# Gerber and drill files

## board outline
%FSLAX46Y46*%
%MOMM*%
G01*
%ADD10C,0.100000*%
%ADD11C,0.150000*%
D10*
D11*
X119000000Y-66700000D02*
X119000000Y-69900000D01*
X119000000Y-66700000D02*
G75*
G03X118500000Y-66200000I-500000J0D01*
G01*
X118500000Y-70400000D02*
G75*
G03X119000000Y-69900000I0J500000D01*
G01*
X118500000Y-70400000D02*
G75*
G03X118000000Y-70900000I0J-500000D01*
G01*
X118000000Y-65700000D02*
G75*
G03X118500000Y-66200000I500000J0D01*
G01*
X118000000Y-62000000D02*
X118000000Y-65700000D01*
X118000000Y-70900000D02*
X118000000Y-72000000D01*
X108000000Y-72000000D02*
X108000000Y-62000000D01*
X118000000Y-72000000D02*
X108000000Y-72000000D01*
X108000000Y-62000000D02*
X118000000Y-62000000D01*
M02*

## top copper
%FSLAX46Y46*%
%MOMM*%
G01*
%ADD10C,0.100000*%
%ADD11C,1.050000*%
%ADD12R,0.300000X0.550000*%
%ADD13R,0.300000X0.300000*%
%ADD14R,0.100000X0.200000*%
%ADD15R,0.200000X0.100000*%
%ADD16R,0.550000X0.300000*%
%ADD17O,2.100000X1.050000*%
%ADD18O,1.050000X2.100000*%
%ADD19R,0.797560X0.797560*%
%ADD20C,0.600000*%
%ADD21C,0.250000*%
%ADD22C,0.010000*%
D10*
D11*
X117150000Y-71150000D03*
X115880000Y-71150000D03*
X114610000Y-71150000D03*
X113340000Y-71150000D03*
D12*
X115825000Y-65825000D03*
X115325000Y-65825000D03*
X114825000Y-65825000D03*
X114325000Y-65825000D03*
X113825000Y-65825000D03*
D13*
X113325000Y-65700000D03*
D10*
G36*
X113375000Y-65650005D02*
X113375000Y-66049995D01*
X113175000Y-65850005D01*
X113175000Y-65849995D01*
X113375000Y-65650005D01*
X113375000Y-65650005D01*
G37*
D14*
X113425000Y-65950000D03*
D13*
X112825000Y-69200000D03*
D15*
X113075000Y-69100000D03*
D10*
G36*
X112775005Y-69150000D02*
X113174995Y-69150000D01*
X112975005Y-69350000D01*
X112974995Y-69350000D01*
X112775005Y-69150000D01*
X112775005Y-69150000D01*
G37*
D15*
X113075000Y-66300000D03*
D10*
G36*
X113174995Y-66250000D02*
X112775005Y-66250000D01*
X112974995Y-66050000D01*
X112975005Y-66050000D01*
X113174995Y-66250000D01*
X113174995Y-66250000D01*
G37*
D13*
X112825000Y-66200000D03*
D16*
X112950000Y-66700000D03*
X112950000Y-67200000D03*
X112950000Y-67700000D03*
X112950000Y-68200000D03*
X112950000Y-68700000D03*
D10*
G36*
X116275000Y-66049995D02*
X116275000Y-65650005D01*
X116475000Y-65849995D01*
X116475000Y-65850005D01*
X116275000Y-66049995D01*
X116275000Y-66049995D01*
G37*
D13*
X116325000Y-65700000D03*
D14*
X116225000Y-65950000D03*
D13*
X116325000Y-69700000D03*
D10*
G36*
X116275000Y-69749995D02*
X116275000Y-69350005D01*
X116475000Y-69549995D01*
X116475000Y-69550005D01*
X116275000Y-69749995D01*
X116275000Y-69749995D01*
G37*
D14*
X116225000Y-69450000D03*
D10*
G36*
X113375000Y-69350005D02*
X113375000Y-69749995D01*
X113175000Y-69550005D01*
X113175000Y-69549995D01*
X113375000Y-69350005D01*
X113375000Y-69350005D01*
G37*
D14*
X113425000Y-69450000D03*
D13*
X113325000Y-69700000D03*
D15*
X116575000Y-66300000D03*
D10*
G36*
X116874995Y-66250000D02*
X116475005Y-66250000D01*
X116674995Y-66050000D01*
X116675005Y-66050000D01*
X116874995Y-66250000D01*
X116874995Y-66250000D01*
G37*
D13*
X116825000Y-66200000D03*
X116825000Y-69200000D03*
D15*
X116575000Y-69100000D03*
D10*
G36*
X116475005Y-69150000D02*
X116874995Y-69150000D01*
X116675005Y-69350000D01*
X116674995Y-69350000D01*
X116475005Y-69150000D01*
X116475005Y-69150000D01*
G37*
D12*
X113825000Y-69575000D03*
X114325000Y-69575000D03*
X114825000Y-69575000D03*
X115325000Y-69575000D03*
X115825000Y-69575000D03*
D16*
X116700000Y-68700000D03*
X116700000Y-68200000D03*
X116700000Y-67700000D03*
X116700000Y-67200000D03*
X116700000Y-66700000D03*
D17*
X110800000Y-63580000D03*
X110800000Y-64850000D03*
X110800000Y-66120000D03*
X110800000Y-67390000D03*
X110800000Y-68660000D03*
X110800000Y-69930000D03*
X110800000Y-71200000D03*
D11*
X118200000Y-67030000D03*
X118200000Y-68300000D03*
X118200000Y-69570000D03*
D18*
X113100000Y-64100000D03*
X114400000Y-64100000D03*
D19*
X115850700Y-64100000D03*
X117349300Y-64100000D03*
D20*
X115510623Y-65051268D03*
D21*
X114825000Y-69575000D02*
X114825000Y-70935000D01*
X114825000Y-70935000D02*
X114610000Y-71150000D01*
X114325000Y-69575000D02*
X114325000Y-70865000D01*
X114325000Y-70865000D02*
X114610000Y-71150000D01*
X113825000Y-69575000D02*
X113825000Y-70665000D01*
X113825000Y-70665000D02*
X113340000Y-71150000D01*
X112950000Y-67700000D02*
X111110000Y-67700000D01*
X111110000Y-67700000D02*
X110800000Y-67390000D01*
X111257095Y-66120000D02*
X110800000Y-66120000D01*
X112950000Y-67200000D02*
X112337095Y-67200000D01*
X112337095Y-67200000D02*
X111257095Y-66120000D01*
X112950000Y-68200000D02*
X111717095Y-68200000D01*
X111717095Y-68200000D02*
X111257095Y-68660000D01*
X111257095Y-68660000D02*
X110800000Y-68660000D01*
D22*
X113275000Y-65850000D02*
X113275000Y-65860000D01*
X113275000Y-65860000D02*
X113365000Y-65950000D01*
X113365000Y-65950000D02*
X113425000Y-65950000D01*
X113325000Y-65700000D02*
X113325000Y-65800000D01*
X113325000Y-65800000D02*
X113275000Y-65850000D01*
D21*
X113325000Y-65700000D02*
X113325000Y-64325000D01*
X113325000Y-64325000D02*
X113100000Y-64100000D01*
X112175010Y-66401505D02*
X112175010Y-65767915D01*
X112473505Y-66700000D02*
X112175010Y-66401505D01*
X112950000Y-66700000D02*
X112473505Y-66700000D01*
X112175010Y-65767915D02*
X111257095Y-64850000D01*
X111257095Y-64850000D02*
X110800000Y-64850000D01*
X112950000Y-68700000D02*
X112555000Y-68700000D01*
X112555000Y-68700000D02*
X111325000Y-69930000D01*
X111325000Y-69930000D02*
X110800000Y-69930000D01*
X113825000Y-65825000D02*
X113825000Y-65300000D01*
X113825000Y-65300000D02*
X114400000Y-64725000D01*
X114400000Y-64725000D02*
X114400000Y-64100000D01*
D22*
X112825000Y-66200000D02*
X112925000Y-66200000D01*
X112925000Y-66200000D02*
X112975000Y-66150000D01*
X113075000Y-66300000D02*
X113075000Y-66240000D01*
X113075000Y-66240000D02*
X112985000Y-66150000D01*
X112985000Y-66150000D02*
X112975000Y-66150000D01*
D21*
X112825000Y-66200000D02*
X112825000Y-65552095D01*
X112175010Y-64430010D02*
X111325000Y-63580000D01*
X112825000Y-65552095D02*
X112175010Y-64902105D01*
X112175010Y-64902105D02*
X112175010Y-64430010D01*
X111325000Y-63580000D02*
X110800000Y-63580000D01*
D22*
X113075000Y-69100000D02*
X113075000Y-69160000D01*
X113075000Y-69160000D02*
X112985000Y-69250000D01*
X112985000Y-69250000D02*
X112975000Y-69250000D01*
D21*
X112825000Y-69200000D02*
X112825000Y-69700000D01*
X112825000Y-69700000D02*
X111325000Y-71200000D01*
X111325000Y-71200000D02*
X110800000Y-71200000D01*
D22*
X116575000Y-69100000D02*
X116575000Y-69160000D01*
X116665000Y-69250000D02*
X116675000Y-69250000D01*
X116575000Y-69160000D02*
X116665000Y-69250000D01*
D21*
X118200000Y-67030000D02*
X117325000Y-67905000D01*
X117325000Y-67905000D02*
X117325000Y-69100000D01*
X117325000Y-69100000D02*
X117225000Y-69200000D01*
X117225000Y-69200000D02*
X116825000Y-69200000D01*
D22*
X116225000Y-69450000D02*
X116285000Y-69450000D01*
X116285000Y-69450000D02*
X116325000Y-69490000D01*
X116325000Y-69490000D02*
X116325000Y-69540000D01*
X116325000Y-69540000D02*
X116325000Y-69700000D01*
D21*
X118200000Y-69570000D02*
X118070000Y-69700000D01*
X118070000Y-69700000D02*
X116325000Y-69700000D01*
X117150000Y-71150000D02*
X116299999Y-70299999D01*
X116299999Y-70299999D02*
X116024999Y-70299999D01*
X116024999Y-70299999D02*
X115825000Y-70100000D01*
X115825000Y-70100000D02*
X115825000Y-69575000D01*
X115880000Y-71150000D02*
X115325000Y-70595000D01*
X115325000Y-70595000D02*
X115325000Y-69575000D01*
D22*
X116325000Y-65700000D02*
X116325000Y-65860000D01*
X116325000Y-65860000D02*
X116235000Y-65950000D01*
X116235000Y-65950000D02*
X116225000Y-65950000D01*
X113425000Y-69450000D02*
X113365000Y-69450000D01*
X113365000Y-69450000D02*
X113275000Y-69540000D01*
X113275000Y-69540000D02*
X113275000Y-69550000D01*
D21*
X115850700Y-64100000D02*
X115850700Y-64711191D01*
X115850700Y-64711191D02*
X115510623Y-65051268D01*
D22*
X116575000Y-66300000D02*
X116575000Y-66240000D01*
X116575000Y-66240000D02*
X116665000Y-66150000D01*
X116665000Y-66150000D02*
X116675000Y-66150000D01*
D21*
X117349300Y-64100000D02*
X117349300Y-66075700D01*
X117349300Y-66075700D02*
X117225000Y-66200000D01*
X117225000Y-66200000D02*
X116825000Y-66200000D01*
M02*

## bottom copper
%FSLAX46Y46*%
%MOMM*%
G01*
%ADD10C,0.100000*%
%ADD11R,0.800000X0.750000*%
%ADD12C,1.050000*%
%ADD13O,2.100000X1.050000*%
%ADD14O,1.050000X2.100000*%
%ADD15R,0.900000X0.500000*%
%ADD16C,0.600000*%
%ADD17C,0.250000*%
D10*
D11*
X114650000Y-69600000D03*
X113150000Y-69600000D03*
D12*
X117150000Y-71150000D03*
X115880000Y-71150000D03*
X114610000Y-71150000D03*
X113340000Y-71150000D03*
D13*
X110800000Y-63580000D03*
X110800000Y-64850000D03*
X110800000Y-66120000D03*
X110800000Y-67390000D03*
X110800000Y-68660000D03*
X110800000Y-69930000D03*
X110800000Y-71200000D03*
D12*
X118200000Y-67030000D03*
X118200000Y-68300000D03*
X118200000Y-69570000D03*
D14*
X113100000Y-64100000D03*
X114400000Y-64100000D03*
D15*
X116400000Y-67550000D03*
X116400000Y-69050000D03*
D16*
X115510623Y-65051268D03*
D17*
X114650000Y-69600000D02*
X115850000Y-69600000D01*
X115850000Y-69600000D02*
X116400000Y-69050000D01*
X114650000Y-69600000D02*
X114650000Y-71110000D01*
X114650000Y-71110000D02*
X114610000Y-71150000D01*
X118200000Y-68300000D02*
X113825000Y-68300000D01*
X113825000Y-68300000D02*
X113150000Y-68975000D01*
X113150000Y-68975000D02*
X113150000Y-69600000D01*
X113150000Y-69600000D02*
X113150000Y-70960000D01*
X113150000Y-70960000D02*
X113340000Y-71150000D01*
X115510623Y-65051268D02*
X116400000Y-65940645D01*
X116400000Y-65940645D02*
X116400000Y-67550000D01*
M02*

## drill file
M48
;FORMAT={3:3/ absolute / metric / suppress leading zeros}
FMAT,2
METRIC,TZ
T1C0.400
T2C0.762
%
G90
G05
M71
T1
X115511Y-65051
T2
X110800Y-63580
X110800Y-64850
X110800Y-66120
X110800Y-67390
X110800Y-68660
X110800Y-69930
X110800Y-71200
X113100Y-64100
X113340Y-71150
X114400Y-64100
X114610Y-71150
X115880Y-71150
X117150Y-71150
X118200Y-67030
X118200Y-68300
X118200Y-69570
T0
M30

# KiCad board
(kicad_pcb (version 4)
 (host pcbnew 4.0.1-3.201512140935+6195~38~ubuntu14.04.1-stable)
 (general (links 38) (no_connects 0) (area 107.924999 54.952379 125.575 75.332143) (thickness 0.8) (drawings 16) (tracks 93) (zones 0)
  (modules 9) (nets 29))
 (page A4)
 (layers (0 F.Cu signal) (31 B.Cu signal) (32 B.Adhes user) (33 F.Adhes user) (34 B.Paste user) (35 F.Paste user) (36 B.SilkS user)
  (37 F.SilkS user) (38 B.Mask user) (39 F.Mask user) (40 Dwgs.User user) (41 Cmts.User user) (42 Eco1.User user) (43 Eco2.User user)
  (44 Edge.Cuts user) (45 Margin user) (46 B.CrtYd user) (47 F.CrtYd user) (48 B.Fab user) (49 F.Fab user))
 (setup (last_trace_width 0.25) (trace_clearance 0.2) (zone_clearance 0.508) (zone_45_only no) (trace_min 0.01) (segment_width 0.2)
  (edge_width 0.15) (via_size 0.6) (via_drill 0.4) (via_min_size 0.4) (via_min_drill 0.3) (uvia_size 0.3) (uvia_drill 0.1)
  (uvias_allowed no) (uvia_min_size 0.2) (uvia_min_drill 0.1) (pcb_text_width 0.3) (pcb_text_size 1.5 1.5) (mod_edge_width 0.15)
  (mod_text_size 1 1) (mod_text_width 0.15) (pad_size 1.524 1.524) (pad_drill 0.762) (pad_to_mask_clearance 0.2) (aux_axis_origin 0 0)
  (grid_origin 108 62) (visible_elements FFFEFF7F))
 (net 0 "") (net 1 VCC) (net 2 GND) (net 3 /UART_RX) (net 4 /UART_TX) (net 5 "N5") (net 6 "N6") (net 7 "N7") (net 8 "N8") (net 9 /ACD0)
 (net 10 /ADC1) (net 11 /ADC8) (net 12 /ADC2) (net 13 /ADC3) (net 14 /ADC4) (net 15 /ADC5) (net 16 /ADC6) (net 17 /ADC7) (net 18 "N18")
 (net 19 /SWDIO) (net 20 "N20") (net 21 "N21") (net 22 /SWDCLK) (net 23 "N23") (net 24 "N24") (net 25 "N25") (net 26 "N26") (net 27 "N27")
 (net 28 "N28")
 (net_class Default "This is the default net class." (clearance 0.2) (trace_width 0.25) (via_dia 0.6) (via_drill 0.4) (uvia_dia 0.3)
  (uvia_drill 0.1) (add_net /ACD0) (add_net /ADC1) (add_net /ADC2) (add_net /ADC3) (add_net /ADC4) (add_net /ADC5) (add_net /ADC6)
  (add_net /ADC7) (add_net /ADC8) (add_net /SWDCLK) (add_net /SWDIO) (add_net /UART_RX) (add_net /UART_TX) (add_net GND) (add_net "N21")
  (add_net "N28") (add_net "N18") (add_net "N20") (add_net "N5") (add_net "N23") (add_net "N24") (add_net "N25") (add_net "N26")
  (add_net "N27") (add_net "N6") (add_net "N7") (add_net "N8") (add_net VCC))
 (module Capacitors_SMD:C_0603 (layer B.Cu) (at 113.9 69.6 180)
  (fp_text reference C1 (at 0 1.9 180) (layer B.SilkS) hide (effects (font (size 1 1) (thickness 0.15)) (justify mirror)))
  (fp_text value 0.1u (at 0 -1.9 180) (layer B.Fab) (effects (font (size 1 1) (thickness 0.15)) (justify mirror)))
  (pad 1 smd rect (at -0.75 0 180) (size 0.8 0.75) (layers B.Cu B.Paste B.Mask) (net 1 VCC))
  (pad 2 smd rect (at 0.75 0 180) (size 0.8 0.75) (layers B.Cu B.Paste B.Mask) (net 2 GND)))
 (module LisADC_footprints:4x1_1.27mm (layer F.Cu) (at 117.15 71.15)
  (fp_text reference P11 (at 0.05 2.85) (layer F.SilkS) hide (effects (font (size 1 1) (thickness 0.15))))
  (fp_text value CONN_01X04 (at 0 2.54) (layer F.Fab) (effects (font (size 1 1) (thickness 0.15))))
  (pad 1 thru_hole circle (at 0 0) (size 1.05 1.05) (drill 0.762) (layers *.Cu *.Mask F.SilkS) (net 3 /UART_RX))
  (pad 2 thru_hole circle (at -1.27 0) (size 1.05 1.05) (drill 0.762) (layers *.Cu *.Mask F.SilkS) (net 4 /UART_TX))
  (pad 3 thru_hole circle (at -2.54 0) (size 1.05 1.05) (drill 0.762) (layers *.Cu *.Mask F.SilkS) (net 1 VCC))
  (pad 4 thru_hole circle (at -3.81 0) (size 1.05 1.05) (drill 0.762) (layers *.Cu *.Mask F.SilkS) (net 2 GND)))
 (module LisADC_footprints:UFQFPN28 (layer F.Cu) (at 114.825 67.7 270)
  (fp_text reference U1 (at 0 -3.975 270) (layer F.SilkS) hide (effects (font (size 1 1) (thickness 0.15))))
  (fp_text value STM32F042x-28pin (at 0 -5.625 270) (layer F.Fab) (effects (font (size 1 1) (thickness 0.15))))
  (pad 2 smd rect (at -1.875 -1 270) (size 0.55 0.3) (layers F.Cu F.Paste F.Mask) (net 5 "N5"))
  (pad 3 smd rect (at -1.875 -0.5 270) (size 0.55 0.3) (layers F.Cu F.Paste F.Mask) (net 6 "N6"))
  (pad 4 smd rect (at -1.875 0 270) (size 0.55 0.3) (layers F.Cu F.Paste F.Mask) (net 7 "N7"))
  (pad 5 smd rect (at -1.875 0.5 270) (size 0.55 0.3) (layers F.Cu F.Paste F.Mask) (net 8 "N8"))
  (pad 6 smd rect (at -1.875 1 270) (size 0.55 0.3) (layers F.Cu F.Paste F.Mask) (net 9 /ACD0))
  (pad 7 smd rect (at -2 1.5) (size 0.3 0.3) (layers F.Cu F.Paste F.Mask) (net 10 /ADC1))
  (pad 7 smd trapezoid (at -1.85 1.55 180) (size 0.2 0.2) (rect_delta 0.19999 0) (layers F.Cu F.Paste F.Mask) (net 10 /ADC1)
   (solder_mask_margin 0.1))
  (pad 7 smd rect (at -1.75 1.4 270) (size 0.2 0.1) (layers F.Cu F.Paste F.Mask) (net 10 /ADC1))
  (pad 14 smd rect (at 1.5 2 90) (size 0.3 0.3) (layers F.Cu F.Paste F.Mask) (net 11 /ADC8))
  (pad 14 smd rect (at 1.4 1.75) (size 0.2 0.1) (layers F.Cu F.Paste F.Mask) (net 11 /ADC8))
  (pad 14 smd trapezoid (at 1.55 1.85 270) (size 0.2 0.2) (rect_delta 0.19999 0) (layers F.Cu F.Paste F.Mask) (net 11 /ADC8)
   (solder_mask_margin 0.1))
  (pad 8 smd rect (at -1.4 1.75) (size 0.2 0.1) (layers F.Cu F.Paste F.Mask) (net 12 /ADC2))
  (pad 8 smd trapezoid (at -1.55 1.85 90) (size 0.2 0.2) (rect_delta 0.19999 0) (layers F.Cu F.Paste F.Mask) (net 12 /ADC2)
   (solder_mask_margin 0.1))
  (pad 8 smd rect (at -1.5 2 90) (size 0.3 0.3) (layers F.Cu F.Paste F.Mask) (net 12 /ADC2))
  (pad 9 smd rect (at -1 1.875) (size 0.55 0.3) (layers F.Cu F.Paste F.Mask) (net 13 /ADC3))
  (pad 10 smd rect (at -0.5 1.875) (size 0.55 0.3) (layers F.Cu F.Paste F.Mask) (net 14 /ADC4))
  (pad 11 smd rect (at 0 1.875) (size 0.55 0.3) (layers F.Cu F.Paste F.Mask) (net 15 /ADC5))
  (pad 12 smd rect (at 0.5 1.875) (size 0.55 0.3) (layers F.Cu F.Paste F.Mask) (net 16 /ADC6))
  (pad 13 smd rect (at 1 1.875) (size 0.55 0.3) (layers F.Cu F.Paste F.Mask) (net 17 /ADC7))
  (pad 1 smd trapezoid (at -1.85 -1.55) (size 0.2 0.2) (rect_delta 0.19999 0) (layers F.Cu F.Paste F.Mask) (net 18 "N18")
   (solder_mask_margin 0.1))
  (pad 1 smd rect (at -2 -1.5) (size 0.3 0.3) (layers F.Cu F.Paste F.Mask) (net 18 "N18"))
  (pad 1 smd rect (at -1.75 -1.4 270) (size 0.2 0.1) (layers F.Cu F.Paste F.Mask) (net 18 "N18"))
  (pad 21 smd rect (at 2 -1.5 180) (size 0.3 0.3) (layers F.Cu F.Paste F.Mask) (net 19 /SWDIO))
  (pad 21 smd trapezoid (at 1.85 -1.55) (size 0.2 0.2) (rect_delta 0.19999 0) (layers F.Cu F.Paste F.Mask) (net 19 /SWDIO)
   (solder_mask_margin 0.1))
  (pad 21 smd rect (at 1.75 -1.4 90) (size 0.2 0.1) (layers F.Cu F.Paste F.Mask) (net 19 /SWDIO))
  (pad 15 smd trapezoid (at 1.85 1.55 180) (size 0.2 0.2) (rect_delta 0.19999 0) (layers F.Cu F.Paste F.Mask) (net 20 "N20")
   (solder_mask_margin 0.1))
  (pad 15 smd rect (at 1.75 1.4 90) (size 0.2 0.1) (layers F.Cu F.Paste F.Mask) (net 20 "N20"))
  (pad 15 smd rect (at 2 1.5 180) (size 0.3 0.3) (layers F.Cu F.Paste F.Mask) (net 20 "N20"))
  (pad 28 smd rect (at -1.4 -1.75 180) (size 0.2 0.1) (layers F.Cu F.Paste F.Mask) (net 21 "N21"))
  (pad 28 smd trapezoid (at -1.55 -1.85 90) (size 0.2 0.2) (rect_delta 0.19999 0) (layers F.Cu F.Paste F.Mask) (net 21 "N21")
   (solder_mask_margin 0.1))
  (pad 28 smd rect (at -1.5 -2 270) (size 0.3 0.3) (layers F.Cu F.Paste F.Mask) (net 21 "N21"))
  (pad 22 smd rect (at 1.5 -2 270) (size 0.3 0.3) (layers F.Cu F.Paste F.Mask) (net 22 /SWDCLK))
  (pad 22 smd rect (at 1.4 -1.75 180) (size 0.2 0.1) (layers F.Cu F.Paste F.Mask) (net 22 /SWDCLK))
  (pad 22 smd trapezoid (at 1.55 -1.85 270) (size 0.2 0.2) (rect_delta 0.19999 0) (layers F.Cu F.Paste F.Mask) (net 22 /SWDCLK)
   (solder_mask_margin 0.1))
  (pad 16 smd rect (at 1.875 1 90) (size 0.55 0.3) (layers F.Cu F.Paste F.Mask) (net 2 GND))
  (pad 17 smd rect (at 1.875 0.5 90) (size 0.55 0.3) (layers F.Cu F.Paste F.Mask) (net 1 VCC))
  (pad 18 smd rect (at 1.875 0 90) (size 0.55 0.3) (layers F.Cu F.Paste F.Mask) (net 1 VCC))
  (pad 19 smd rect (at 1.875 -0.5 90) (size 0.55 0.3) (layers F.Cu F.Paste F.Mask) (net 4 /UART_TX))
  (pad 20 smd rect (at 1.875 -1 90) (size 0.55 0.3) (layers F.Cu F.Paste F.Mask) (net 3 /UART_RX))
  (pad 23 smd rect (at 1 -1.875 180) (size 0.55 0.3) (layers F.Cu F.Paste F.Mask) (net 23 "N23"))
  (pad 24 smd rect (at 0.5 -1.875 180) (size 0.55 0.3) (layers F.Cu F.Paste F.Mask) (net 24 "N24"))
  (pad 25 smd rect (at 0 -1.875 180) (size 0.55 0.3) (layers F.Cu F.Paste F.Mask) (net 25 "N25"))
  (pad 26 smd rect (at -0.5 -1.875 180) (size 0.55 0.3) (layers F.Cu F.Paste F.Mask) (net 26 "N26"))
  (pad 27 smd rect (at -1 -1.875 180) (size 0.55 0.3) (layers F.Cu F.Paste F.Mask) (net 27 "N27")))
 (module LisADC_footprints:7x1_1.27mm (layer F.Cu) (at 110.8 63.58 90)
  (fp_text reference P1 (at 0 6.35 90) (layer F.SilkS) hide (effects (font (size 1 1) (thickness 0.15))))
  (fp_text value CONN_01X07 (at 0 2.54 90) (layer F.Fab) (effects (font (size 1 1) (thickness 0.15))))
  (pad 1 thru_hole oval (at 0 0 90) (size 1.05 2.1) (drill 0.762) (layers *.Cu *.Mask F.SilkS) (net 12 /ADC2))
  (pad 2 thru_hole oval (at -1.27 0 90) (size 1.05 2.1) (drill 0.762) (layers *.Cu *.Mask F.SilkS) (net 13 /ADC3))
  (pad 3 thru_hole oval (at -2.54 0 90) (size 1.05 2.1) (drill 0.762) (layers *.Cu *.Mask F.SilkS) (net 14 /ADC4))
  (pad 4 thru_hole oval (at -3.81 0 90) (size 1.05 2.1) (drill 0.762) (layers *.Cu *.Mask F.SilkS) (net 15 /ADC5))
  (pad 5 thru_hole oval (at -5.08 0 90) (size 1.05 2.1) (drill 0.762) (layers *.Cu *.Mask F.SilkS) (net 16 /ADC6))
  (pad 6 thru_hole oval (at -6.35 0 90) (size 1.05 2.1) (drill 0.762) (layers *.Cu *.Mask F.SilkS) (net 17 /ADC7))
  (pad 7 thru_hole oval (at -7.62 0 90) (size 1.05 2.1) (drill 0.762) (layers *.Cu *.Mask F.SilkS) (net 11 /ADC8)))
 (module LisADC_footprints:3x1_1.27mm (layer F.Cu) (at 118.25 68.305 90)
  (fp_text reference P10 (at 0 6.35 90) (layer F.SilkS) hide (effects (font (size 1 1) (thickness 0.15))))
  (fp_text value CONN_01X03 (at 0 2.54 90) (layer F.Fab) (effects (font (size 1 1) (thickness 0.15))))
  (pad 1 thru_hole circle (at 1.275 -0.05 90) (size 1.05 1.05) (drill 0.762) (layers *.Cu *.Mask F.SilkS) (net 22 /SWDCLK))
  (pad 2 thru_hole circle (at 0.005 -0.05 90) (size 1.05 1.05) (drill 0.762) (layers *.Cu *.Mask F.SilkS) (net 2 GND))
  (pad 3 thru_hole circle (at -1.265 -0.05 90) (size 1.05 1.05) (drill 0.762) (layers *.Cu *.Mask F.SilkS) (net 19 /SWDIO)))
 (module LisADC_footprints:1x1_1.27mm (layer F.Cu) (at 113.1 64.1)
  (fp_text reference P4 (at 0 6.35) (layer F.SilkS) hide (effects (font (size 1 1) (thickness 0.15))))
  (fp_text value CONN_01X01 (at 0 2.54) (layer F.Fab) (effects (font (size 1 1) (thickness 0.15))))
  (pad 1 thru_hole oval (at 0 0) (size 1.05 2.1) (drill 0.762) (layers *.Cu *.Mask F.SilkS) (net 10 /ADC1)))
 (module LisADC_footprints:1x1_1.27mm (layer F.Cu) (at 114.4 64.1)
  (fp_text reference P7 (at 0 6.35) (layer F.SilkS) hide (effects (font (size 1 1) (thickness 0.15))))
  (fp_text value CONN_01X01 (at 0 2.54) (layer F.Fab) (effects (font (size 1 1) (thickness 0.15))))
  (pad 1 thru_hole oval (at 0 0) (size 1.05 2.1) (drill 0.762) (layers *.Cu *.Mask F.SilkS) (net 9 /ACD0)))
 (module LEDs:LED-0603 (layer F.Cu) (at 116.6 64.1 180)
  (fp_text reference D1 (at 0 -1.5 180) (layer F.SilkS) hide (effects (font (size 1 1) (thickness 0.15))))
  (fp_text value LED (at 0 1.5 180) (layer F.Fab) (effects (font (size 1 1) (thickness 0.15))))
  (pad 2 smd rect (at 0.7493 0) (size 0.79756 0.79756) (layers F.Cu F.Paste F.Mask) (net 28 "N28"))
  (pad 1 smd rect (at -0.7493 0) (size 0.79756 0.79756) (layers F.Cu F.Paste F.Mask) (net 21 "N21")))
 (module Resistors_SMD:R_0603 (layer B.Cu) (at 116.4 68.3 270)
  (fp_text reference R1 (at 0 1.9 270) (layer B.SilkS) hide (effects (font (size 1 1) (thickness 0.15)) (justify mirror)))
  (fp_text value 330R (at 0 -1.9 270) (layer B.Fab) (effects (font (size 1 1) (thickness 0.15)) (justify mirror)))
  (pad 1 smd rect (at -0.75 0 270) (size 0.5 0.9) (layers B.Cu B.Paste B.Mask) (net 28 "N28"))
  (pad 2 smd rect (at 0.75 0 270) (size 0.5 0.9) (layers B.Cu B.Paste B.Mask) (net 1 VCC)))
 (gr_line (start 119 66.7) (end 119 69.9) (layer Edge.Cuts) (width 0.15))
 (gr_arc (start 118.5 66.7) (end 118.5 66.2) (angle 90) (layer Edge.Cuts) (width 0.15))
 (gr_arc (start 118.5 69.9) (end 119 69.9) (angle 90) (layer Edge.Cuts) (width 0.15))
 (gr_arc (start 118.5 70.9) (end 118 70.9) (angle 90) (layer Edge.Cuts) (width 0.15))
 (gr_arc (start 118.5 65.7) (end 118.5 66.2) (angle 90) (layer Edge.Cuts) (width 0.15))
 (gr_line (start 118 62) (end 118 65.7) (layer Edge.Cuts) (width 0.15))
 (gr_line (start 118 70.9) (end 118 72) (layer Edge.Cuts) (width 0.15))
 (gr_line (start 108 72) (end 108 62) (layer Edge.Cuts) (width 0.15))
 (gr_line (start 118 72) (end 108 72) (layer Edge.Cuts) (width 0.15))
 (gr_line (start 108 62) (end 118 62) (layer Edge.Cuts) (width 0.15))
 (segment (start 114.65 69.6) (end 115.85 69.6) (width 0.25) (layer B.Cu) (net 1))
 (segment (start 115.85 69.6) (end 116.4 69.05) (width 0.25) (layer B.Cu) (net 1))
 (segment (start 114.825 69.575) (end 114.825 70.935) (width 0.25) (layer F.Cu) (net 1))
 (segment (start 114.825 70.935) (end 114.61 71.15) (width 0.25) (layer F.Cu) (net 1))
 (segment (start 114.325 69.575) (end 114.325 70.865) (width 0.25) (layer F.Cu) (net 1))
 (segment (start 114.325 70.865) (end 114.61 71.15) (width 0.25) (layer F.Cu) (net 1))
 (segment (start 114.65 69.6) (end 114.65 71.11) (width 0.25) (layer B.Cu) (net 1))
 (segment (start 114.65 71.11) (end 114.61 71.15) (width 0.25) (layer B.Cu) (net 1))
 (segment (start 118.2 68.3) (end 113.825 68.3) (width 0.25) (layer B.Cu) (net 2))
 (segment (start 113.825 68.3) (end 113.15 68.975) (width 0.25) (layer B.Cu) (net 2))
 (segment (start 113.15 68.975) (end 113.15 69.6) (width 0.25) (layer B.Cu) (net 2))
 (segment (start 113.825 69.575) (end 113.825 70.665) (width 0.25) (layer F.Cu) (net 2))
 (segment (start 113.825 70.665) (end 113.34 71.15) (width 0.25) (layer F.Cu) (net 2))
 (segment (start 113.15 69.6) (end 113.15 70.96) (width 0.25) (layer B.Cu) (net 2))
 (segment (start 113.15 70.96) (end 113.34 71.15) (width 0.25) (layer B.Cu) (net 2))
 (segment (start 112.95 67.7) (end 111.11 67.7) (width 0.25) (layer F.Cu) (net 15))
 (segment (start 111.11 67.7) (end 110.8 67.39) (width 0.25) (layer F.Cu) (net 15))
 (segment (start 111.257095 66.12) (end 110.8 66.12) (width 0.25) (layer F.Cu) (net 14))
 (segment (start 112.95 67.2) (end 112.337095 67.2) (width 0.25) (layer F.Cu) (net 14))
 (segment (start 112.337095 67.2) (end 111.257095 66.12) (width 0.25) (layer F.Cu) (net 14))
 (segment (start 112.95 68.2) (end 111.717095 68.2) (width 0.25) (layer F.Cu) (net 16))
 (segment (start 111.717095 68.2) (end 111.257095 68.66) (width 0.25) (layer F.Cu) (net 16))
 (segment (start 111.257095 68.66) (end 110.8 68.66) (width 0.25) (layer F.Cu) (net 16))
 (segment (start 113.275 65.85) (end 113.275 65.86) (width 0.01) (layer F.Cu) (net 10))
 (segment (start 113.275 65.86) (end 113.365 65.95) (width 0.01) (layer F.Cu) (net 10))
 (segment (start 113.365 65.95) (end 113.425 65.95) (width 0.01) (layer F.Cu) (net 10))
 (segment (start 113.325 65.7) (end 113.325 65.8) (width 0.01) (layer F.Cu) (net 10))
 (segment (start 113.325 65.8) (end 113.275 65.85) (width 0.01) (layer F.Cu) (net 10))
 (segment (start 113.325 65.7) (end 113.325 64.325) (width 0.25) (layer F.Cu) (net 10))
 (segment (start 113.325 64.325) (end 113.1 64.1) (width 0.25) (layer F.Cu) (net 10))
 (segment (start 112.17501 66.401505) (end 112.17501 65.767915) (width 0.25) (layer F.Cu) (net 13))
 (segment (start 112.473505 66.7) (end 112.17501 66.401505) (width 0.25) (layer F.Cu) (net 13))
 (segment (start 112.95 66.7) (end 112.473505 66.7) (width 0.25) (layer F.Cu) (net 13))
 (segment (start 112.17501 65.767915) (end 111.257095 64.85) (width 0.25) (layer F.Cu) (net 13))
 (segment (start 111.257095 64.85) (end 110.8 64.85) (width 0.25) (layer F.Cu) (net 13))
 (segment (start 112.95 68.7) (end 112.555 68.7) (width 0.25) (layer F.Cu) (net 17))
 (segment (start 112.555 68.7) (end 111.325 69.93) (width 0.25) (layer F.Cu) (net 17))
 (segment (start 111.325 69.93) (end 110.8 69.93) (width 0.25) (layer F.Cu) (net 17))
 (segment (start 113.825 65.825) (end 113.825 65.3) (width 0.25) (layer F.Cu) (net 9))
 (segment (start 113.825 65.3) (end 114.4 64.725) (width 0.25) (layer F.Cu) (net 9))
 (segment (start 114.4 64.725) (end 114.4 64.1) (width 0.25) (layer F.Cu) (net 9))
 (segment (start 112.825 66.2) (end 112.925 66.2) (width 0.01) (layer F.Cu) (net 12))
 (segment (start 112.925 66.2) (end 112.975 66.15) (width 0.01) (layer F.Cu) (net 12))
 (segment (start 113.075 66.3) (end 113.075 66.24) (width 0.01) (layer F.Cu) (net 12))
 (segment (start 113.075 66.24) (end 112.985 66.15) (width 0.01) (layer F.Cu) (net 12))
 (segment (start 112.985 66.15) (end 112.975 66.15) (width 0.01) (layer F.Cu) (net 12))
 (segment (start 112.825 66.2) (end 112.825 65.552095) (width 0.25) (layer F.Cu) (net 12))
 (segment (start 112.17501 64.43001) (end 111.325 63.58) (width 0.25) (layer F.Cu) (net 12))
 (segment (start 112.825 65.552095) (end 112.17501 64.902105) (width 0.25) (layer F.Cu) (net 12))
 (segment (start 112.17501 64.902105) (end 112.17501 64.43001) (width 0.25) (layer F.Cu) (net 12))
 (segment (start 111.325 63.58) (end 110.8 63.58) (width 0.25) (layer F.Cu) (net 12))
 (segment (start 113.075 69.1) (end 113.075 69.16) (width 0.01) (layer F.Cu) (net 11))
 (segment (start 113.075 69.16) (end 112.985 69.25) (width 0.01) (layer F.Cu) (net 11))
 (segment (start 112.985 69.25) (end 112.975 69.25) (width 0.01) (layer F.Cu) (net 11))
 (segment (start 112.825 69.2) (end 112.825 69.7) (width 0.25) (layer F.Cu) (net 11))
 (segment (start 112.825 69.7) (end 111.325 71.2) (width 0.25) (layer F.Cu) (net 11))
 (segment (start 111.325 71.2) (end 110.8 71.2) (width 0.25) (layer F.Cu) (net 11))
 (segment (start 116.575 69.1) (end 116.575 69.16) (width 0.01) (layer F.Cu) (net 22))
 (segment (start 116.665 69.25) (end 116.675 69.25) (width 0.01) (layer F.Cu) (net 22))
 (segment (start 116.575 69.16) (end 116.665 69.25) (width 0.01) (layer F.Cu) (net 22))
 (segment (start 118.2 67.03) (end 117.325 67.905) (width 0.25) (layer F.Cu) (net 22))
 (segment (start 117.325 67.905) (end 117.325 69.1) (width 0.25) (layer F.Cu) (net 22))
 (segment (start 117.325 69.1) (end 117.225 69.2) (width 0.25) (layer F.Cu) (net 22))
 (segment (start 117.225 69.2) (end 116.825 69.2) (width 0.25) (layer F.Cu) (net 22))
 (segment (start 116.225 69.45) (end 116.285 69.45) (width 0.01) (layer F.Cu) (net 19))
 (segment (start 116.285 69.45) (end 116.325 69.49) (width 0.01) (layer F.Cu) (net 19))
 (segment (start 116.325 69.49) (end 116.325 69.54) (width 0.01) (layer F.Cu) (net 19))
 (segment (start 116.325 69.54) (end 116.325 69.7) (width 0.01) (layer F.Cu) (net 19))
 (segment (start 118.2 69.57) (end 118.07 69.7) (width 0.25) (layer F.Cu) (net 19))
 (segment (start 118.07 69.7) (end 116.325 69.7) (width 0.25) (layer F.Cu) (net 19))
 (segment (start 117.15 71.15) (end 116.299999 70.299999) (width 0.25) (layer F.Cu) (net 3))
 (segment (start 116.299999 70.299999) (end 116.024999 70.299999) (width 0.25) (layer F.Cu) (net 3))
 (segment (start 116.024999 70.299999) (end 115.825 70.1) (width 0.25) (layer F.Cu) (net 3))
 (segment (start 115.825 70.1) (end 115.825 69.575) (width 0.25) (layer F.Cu) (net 3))
 (segment (start 115.88 71.15) (end 115.325 70.595) (width 0.25) (layer F.Cu) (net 4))
 (segment (start 115.325 70.595) (end 115.325 69.575) (width 0.25) (layer F.Cu) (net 4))
 (segment (start 116.325 65.7) (end 116.325 65.86) (width 0.01) (layer F.Cu) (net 18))
 (segment (start 116.325 65.86) (end 116.235 65.95) (width 0.01) (layer F.Cu) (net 18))
 (segment (start 116.235 65.95) (end 116.225 65.95) (width 0.01) (layer F.Cu) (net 18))
 (segment (start 113.425 69.45) (end 113.365 69.45) (width 0.01) (layer F.Cu) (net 20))
 (segment (start 113.365 69.45) (end 113.275 69.54) (width 0.01) (layer F.Cu) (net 20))
 (segment (start 113.275 69.54) (end 113.275 69.55) (width 0.01) (layer F.Cu) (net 20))
 (segment (start 115.510623 65.051268) (end 116.4 65.940645) (width 0.25) (layer B.Cu) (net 28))
 (segment (start 116.4 65.940645) (end 116.4 67.55) (width 0.25) (layer B.Cu) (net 28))
 (segment (start 115.8507 64.1) (end 115.8507 64.711191) (width 0.25) (layer F.Cu) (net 28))
 (segment (start 115.8507 64.711191) (end 115.510623 65.051268) (width 0.25) (layer F.Cu) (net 28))
 (via (at 115.510623 65.051268) (size 0.6) (drill 0.4) (layers F.Cu B.Cu) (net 28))
 (segment (start 116.575 66.3) (end 116.575 66.24) (width 0.01) (layer F.Cu) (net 21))
 (segment (start 116.575 66.24) (end 116.665 66.15) (width 0.01) (layer F.Cu) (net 21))
 (segment (start 116.665 66.15) (end 116.675 66.15) (width 0.01) (layer F.Cu) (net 21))
 (segment (start 117.3493 64.1) (end 117.3493 66.0757) (width 0.25) (layer F.Cu) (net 21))
 (segment (start 117.3493 66.0757) (end 117.225 66.2) (width 0.25) (layer F.Cu) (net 21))
 (segment (start 117.225 66.2) (end 116.825 66.2) (width 0.25) (layer F.Cu) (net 21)))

